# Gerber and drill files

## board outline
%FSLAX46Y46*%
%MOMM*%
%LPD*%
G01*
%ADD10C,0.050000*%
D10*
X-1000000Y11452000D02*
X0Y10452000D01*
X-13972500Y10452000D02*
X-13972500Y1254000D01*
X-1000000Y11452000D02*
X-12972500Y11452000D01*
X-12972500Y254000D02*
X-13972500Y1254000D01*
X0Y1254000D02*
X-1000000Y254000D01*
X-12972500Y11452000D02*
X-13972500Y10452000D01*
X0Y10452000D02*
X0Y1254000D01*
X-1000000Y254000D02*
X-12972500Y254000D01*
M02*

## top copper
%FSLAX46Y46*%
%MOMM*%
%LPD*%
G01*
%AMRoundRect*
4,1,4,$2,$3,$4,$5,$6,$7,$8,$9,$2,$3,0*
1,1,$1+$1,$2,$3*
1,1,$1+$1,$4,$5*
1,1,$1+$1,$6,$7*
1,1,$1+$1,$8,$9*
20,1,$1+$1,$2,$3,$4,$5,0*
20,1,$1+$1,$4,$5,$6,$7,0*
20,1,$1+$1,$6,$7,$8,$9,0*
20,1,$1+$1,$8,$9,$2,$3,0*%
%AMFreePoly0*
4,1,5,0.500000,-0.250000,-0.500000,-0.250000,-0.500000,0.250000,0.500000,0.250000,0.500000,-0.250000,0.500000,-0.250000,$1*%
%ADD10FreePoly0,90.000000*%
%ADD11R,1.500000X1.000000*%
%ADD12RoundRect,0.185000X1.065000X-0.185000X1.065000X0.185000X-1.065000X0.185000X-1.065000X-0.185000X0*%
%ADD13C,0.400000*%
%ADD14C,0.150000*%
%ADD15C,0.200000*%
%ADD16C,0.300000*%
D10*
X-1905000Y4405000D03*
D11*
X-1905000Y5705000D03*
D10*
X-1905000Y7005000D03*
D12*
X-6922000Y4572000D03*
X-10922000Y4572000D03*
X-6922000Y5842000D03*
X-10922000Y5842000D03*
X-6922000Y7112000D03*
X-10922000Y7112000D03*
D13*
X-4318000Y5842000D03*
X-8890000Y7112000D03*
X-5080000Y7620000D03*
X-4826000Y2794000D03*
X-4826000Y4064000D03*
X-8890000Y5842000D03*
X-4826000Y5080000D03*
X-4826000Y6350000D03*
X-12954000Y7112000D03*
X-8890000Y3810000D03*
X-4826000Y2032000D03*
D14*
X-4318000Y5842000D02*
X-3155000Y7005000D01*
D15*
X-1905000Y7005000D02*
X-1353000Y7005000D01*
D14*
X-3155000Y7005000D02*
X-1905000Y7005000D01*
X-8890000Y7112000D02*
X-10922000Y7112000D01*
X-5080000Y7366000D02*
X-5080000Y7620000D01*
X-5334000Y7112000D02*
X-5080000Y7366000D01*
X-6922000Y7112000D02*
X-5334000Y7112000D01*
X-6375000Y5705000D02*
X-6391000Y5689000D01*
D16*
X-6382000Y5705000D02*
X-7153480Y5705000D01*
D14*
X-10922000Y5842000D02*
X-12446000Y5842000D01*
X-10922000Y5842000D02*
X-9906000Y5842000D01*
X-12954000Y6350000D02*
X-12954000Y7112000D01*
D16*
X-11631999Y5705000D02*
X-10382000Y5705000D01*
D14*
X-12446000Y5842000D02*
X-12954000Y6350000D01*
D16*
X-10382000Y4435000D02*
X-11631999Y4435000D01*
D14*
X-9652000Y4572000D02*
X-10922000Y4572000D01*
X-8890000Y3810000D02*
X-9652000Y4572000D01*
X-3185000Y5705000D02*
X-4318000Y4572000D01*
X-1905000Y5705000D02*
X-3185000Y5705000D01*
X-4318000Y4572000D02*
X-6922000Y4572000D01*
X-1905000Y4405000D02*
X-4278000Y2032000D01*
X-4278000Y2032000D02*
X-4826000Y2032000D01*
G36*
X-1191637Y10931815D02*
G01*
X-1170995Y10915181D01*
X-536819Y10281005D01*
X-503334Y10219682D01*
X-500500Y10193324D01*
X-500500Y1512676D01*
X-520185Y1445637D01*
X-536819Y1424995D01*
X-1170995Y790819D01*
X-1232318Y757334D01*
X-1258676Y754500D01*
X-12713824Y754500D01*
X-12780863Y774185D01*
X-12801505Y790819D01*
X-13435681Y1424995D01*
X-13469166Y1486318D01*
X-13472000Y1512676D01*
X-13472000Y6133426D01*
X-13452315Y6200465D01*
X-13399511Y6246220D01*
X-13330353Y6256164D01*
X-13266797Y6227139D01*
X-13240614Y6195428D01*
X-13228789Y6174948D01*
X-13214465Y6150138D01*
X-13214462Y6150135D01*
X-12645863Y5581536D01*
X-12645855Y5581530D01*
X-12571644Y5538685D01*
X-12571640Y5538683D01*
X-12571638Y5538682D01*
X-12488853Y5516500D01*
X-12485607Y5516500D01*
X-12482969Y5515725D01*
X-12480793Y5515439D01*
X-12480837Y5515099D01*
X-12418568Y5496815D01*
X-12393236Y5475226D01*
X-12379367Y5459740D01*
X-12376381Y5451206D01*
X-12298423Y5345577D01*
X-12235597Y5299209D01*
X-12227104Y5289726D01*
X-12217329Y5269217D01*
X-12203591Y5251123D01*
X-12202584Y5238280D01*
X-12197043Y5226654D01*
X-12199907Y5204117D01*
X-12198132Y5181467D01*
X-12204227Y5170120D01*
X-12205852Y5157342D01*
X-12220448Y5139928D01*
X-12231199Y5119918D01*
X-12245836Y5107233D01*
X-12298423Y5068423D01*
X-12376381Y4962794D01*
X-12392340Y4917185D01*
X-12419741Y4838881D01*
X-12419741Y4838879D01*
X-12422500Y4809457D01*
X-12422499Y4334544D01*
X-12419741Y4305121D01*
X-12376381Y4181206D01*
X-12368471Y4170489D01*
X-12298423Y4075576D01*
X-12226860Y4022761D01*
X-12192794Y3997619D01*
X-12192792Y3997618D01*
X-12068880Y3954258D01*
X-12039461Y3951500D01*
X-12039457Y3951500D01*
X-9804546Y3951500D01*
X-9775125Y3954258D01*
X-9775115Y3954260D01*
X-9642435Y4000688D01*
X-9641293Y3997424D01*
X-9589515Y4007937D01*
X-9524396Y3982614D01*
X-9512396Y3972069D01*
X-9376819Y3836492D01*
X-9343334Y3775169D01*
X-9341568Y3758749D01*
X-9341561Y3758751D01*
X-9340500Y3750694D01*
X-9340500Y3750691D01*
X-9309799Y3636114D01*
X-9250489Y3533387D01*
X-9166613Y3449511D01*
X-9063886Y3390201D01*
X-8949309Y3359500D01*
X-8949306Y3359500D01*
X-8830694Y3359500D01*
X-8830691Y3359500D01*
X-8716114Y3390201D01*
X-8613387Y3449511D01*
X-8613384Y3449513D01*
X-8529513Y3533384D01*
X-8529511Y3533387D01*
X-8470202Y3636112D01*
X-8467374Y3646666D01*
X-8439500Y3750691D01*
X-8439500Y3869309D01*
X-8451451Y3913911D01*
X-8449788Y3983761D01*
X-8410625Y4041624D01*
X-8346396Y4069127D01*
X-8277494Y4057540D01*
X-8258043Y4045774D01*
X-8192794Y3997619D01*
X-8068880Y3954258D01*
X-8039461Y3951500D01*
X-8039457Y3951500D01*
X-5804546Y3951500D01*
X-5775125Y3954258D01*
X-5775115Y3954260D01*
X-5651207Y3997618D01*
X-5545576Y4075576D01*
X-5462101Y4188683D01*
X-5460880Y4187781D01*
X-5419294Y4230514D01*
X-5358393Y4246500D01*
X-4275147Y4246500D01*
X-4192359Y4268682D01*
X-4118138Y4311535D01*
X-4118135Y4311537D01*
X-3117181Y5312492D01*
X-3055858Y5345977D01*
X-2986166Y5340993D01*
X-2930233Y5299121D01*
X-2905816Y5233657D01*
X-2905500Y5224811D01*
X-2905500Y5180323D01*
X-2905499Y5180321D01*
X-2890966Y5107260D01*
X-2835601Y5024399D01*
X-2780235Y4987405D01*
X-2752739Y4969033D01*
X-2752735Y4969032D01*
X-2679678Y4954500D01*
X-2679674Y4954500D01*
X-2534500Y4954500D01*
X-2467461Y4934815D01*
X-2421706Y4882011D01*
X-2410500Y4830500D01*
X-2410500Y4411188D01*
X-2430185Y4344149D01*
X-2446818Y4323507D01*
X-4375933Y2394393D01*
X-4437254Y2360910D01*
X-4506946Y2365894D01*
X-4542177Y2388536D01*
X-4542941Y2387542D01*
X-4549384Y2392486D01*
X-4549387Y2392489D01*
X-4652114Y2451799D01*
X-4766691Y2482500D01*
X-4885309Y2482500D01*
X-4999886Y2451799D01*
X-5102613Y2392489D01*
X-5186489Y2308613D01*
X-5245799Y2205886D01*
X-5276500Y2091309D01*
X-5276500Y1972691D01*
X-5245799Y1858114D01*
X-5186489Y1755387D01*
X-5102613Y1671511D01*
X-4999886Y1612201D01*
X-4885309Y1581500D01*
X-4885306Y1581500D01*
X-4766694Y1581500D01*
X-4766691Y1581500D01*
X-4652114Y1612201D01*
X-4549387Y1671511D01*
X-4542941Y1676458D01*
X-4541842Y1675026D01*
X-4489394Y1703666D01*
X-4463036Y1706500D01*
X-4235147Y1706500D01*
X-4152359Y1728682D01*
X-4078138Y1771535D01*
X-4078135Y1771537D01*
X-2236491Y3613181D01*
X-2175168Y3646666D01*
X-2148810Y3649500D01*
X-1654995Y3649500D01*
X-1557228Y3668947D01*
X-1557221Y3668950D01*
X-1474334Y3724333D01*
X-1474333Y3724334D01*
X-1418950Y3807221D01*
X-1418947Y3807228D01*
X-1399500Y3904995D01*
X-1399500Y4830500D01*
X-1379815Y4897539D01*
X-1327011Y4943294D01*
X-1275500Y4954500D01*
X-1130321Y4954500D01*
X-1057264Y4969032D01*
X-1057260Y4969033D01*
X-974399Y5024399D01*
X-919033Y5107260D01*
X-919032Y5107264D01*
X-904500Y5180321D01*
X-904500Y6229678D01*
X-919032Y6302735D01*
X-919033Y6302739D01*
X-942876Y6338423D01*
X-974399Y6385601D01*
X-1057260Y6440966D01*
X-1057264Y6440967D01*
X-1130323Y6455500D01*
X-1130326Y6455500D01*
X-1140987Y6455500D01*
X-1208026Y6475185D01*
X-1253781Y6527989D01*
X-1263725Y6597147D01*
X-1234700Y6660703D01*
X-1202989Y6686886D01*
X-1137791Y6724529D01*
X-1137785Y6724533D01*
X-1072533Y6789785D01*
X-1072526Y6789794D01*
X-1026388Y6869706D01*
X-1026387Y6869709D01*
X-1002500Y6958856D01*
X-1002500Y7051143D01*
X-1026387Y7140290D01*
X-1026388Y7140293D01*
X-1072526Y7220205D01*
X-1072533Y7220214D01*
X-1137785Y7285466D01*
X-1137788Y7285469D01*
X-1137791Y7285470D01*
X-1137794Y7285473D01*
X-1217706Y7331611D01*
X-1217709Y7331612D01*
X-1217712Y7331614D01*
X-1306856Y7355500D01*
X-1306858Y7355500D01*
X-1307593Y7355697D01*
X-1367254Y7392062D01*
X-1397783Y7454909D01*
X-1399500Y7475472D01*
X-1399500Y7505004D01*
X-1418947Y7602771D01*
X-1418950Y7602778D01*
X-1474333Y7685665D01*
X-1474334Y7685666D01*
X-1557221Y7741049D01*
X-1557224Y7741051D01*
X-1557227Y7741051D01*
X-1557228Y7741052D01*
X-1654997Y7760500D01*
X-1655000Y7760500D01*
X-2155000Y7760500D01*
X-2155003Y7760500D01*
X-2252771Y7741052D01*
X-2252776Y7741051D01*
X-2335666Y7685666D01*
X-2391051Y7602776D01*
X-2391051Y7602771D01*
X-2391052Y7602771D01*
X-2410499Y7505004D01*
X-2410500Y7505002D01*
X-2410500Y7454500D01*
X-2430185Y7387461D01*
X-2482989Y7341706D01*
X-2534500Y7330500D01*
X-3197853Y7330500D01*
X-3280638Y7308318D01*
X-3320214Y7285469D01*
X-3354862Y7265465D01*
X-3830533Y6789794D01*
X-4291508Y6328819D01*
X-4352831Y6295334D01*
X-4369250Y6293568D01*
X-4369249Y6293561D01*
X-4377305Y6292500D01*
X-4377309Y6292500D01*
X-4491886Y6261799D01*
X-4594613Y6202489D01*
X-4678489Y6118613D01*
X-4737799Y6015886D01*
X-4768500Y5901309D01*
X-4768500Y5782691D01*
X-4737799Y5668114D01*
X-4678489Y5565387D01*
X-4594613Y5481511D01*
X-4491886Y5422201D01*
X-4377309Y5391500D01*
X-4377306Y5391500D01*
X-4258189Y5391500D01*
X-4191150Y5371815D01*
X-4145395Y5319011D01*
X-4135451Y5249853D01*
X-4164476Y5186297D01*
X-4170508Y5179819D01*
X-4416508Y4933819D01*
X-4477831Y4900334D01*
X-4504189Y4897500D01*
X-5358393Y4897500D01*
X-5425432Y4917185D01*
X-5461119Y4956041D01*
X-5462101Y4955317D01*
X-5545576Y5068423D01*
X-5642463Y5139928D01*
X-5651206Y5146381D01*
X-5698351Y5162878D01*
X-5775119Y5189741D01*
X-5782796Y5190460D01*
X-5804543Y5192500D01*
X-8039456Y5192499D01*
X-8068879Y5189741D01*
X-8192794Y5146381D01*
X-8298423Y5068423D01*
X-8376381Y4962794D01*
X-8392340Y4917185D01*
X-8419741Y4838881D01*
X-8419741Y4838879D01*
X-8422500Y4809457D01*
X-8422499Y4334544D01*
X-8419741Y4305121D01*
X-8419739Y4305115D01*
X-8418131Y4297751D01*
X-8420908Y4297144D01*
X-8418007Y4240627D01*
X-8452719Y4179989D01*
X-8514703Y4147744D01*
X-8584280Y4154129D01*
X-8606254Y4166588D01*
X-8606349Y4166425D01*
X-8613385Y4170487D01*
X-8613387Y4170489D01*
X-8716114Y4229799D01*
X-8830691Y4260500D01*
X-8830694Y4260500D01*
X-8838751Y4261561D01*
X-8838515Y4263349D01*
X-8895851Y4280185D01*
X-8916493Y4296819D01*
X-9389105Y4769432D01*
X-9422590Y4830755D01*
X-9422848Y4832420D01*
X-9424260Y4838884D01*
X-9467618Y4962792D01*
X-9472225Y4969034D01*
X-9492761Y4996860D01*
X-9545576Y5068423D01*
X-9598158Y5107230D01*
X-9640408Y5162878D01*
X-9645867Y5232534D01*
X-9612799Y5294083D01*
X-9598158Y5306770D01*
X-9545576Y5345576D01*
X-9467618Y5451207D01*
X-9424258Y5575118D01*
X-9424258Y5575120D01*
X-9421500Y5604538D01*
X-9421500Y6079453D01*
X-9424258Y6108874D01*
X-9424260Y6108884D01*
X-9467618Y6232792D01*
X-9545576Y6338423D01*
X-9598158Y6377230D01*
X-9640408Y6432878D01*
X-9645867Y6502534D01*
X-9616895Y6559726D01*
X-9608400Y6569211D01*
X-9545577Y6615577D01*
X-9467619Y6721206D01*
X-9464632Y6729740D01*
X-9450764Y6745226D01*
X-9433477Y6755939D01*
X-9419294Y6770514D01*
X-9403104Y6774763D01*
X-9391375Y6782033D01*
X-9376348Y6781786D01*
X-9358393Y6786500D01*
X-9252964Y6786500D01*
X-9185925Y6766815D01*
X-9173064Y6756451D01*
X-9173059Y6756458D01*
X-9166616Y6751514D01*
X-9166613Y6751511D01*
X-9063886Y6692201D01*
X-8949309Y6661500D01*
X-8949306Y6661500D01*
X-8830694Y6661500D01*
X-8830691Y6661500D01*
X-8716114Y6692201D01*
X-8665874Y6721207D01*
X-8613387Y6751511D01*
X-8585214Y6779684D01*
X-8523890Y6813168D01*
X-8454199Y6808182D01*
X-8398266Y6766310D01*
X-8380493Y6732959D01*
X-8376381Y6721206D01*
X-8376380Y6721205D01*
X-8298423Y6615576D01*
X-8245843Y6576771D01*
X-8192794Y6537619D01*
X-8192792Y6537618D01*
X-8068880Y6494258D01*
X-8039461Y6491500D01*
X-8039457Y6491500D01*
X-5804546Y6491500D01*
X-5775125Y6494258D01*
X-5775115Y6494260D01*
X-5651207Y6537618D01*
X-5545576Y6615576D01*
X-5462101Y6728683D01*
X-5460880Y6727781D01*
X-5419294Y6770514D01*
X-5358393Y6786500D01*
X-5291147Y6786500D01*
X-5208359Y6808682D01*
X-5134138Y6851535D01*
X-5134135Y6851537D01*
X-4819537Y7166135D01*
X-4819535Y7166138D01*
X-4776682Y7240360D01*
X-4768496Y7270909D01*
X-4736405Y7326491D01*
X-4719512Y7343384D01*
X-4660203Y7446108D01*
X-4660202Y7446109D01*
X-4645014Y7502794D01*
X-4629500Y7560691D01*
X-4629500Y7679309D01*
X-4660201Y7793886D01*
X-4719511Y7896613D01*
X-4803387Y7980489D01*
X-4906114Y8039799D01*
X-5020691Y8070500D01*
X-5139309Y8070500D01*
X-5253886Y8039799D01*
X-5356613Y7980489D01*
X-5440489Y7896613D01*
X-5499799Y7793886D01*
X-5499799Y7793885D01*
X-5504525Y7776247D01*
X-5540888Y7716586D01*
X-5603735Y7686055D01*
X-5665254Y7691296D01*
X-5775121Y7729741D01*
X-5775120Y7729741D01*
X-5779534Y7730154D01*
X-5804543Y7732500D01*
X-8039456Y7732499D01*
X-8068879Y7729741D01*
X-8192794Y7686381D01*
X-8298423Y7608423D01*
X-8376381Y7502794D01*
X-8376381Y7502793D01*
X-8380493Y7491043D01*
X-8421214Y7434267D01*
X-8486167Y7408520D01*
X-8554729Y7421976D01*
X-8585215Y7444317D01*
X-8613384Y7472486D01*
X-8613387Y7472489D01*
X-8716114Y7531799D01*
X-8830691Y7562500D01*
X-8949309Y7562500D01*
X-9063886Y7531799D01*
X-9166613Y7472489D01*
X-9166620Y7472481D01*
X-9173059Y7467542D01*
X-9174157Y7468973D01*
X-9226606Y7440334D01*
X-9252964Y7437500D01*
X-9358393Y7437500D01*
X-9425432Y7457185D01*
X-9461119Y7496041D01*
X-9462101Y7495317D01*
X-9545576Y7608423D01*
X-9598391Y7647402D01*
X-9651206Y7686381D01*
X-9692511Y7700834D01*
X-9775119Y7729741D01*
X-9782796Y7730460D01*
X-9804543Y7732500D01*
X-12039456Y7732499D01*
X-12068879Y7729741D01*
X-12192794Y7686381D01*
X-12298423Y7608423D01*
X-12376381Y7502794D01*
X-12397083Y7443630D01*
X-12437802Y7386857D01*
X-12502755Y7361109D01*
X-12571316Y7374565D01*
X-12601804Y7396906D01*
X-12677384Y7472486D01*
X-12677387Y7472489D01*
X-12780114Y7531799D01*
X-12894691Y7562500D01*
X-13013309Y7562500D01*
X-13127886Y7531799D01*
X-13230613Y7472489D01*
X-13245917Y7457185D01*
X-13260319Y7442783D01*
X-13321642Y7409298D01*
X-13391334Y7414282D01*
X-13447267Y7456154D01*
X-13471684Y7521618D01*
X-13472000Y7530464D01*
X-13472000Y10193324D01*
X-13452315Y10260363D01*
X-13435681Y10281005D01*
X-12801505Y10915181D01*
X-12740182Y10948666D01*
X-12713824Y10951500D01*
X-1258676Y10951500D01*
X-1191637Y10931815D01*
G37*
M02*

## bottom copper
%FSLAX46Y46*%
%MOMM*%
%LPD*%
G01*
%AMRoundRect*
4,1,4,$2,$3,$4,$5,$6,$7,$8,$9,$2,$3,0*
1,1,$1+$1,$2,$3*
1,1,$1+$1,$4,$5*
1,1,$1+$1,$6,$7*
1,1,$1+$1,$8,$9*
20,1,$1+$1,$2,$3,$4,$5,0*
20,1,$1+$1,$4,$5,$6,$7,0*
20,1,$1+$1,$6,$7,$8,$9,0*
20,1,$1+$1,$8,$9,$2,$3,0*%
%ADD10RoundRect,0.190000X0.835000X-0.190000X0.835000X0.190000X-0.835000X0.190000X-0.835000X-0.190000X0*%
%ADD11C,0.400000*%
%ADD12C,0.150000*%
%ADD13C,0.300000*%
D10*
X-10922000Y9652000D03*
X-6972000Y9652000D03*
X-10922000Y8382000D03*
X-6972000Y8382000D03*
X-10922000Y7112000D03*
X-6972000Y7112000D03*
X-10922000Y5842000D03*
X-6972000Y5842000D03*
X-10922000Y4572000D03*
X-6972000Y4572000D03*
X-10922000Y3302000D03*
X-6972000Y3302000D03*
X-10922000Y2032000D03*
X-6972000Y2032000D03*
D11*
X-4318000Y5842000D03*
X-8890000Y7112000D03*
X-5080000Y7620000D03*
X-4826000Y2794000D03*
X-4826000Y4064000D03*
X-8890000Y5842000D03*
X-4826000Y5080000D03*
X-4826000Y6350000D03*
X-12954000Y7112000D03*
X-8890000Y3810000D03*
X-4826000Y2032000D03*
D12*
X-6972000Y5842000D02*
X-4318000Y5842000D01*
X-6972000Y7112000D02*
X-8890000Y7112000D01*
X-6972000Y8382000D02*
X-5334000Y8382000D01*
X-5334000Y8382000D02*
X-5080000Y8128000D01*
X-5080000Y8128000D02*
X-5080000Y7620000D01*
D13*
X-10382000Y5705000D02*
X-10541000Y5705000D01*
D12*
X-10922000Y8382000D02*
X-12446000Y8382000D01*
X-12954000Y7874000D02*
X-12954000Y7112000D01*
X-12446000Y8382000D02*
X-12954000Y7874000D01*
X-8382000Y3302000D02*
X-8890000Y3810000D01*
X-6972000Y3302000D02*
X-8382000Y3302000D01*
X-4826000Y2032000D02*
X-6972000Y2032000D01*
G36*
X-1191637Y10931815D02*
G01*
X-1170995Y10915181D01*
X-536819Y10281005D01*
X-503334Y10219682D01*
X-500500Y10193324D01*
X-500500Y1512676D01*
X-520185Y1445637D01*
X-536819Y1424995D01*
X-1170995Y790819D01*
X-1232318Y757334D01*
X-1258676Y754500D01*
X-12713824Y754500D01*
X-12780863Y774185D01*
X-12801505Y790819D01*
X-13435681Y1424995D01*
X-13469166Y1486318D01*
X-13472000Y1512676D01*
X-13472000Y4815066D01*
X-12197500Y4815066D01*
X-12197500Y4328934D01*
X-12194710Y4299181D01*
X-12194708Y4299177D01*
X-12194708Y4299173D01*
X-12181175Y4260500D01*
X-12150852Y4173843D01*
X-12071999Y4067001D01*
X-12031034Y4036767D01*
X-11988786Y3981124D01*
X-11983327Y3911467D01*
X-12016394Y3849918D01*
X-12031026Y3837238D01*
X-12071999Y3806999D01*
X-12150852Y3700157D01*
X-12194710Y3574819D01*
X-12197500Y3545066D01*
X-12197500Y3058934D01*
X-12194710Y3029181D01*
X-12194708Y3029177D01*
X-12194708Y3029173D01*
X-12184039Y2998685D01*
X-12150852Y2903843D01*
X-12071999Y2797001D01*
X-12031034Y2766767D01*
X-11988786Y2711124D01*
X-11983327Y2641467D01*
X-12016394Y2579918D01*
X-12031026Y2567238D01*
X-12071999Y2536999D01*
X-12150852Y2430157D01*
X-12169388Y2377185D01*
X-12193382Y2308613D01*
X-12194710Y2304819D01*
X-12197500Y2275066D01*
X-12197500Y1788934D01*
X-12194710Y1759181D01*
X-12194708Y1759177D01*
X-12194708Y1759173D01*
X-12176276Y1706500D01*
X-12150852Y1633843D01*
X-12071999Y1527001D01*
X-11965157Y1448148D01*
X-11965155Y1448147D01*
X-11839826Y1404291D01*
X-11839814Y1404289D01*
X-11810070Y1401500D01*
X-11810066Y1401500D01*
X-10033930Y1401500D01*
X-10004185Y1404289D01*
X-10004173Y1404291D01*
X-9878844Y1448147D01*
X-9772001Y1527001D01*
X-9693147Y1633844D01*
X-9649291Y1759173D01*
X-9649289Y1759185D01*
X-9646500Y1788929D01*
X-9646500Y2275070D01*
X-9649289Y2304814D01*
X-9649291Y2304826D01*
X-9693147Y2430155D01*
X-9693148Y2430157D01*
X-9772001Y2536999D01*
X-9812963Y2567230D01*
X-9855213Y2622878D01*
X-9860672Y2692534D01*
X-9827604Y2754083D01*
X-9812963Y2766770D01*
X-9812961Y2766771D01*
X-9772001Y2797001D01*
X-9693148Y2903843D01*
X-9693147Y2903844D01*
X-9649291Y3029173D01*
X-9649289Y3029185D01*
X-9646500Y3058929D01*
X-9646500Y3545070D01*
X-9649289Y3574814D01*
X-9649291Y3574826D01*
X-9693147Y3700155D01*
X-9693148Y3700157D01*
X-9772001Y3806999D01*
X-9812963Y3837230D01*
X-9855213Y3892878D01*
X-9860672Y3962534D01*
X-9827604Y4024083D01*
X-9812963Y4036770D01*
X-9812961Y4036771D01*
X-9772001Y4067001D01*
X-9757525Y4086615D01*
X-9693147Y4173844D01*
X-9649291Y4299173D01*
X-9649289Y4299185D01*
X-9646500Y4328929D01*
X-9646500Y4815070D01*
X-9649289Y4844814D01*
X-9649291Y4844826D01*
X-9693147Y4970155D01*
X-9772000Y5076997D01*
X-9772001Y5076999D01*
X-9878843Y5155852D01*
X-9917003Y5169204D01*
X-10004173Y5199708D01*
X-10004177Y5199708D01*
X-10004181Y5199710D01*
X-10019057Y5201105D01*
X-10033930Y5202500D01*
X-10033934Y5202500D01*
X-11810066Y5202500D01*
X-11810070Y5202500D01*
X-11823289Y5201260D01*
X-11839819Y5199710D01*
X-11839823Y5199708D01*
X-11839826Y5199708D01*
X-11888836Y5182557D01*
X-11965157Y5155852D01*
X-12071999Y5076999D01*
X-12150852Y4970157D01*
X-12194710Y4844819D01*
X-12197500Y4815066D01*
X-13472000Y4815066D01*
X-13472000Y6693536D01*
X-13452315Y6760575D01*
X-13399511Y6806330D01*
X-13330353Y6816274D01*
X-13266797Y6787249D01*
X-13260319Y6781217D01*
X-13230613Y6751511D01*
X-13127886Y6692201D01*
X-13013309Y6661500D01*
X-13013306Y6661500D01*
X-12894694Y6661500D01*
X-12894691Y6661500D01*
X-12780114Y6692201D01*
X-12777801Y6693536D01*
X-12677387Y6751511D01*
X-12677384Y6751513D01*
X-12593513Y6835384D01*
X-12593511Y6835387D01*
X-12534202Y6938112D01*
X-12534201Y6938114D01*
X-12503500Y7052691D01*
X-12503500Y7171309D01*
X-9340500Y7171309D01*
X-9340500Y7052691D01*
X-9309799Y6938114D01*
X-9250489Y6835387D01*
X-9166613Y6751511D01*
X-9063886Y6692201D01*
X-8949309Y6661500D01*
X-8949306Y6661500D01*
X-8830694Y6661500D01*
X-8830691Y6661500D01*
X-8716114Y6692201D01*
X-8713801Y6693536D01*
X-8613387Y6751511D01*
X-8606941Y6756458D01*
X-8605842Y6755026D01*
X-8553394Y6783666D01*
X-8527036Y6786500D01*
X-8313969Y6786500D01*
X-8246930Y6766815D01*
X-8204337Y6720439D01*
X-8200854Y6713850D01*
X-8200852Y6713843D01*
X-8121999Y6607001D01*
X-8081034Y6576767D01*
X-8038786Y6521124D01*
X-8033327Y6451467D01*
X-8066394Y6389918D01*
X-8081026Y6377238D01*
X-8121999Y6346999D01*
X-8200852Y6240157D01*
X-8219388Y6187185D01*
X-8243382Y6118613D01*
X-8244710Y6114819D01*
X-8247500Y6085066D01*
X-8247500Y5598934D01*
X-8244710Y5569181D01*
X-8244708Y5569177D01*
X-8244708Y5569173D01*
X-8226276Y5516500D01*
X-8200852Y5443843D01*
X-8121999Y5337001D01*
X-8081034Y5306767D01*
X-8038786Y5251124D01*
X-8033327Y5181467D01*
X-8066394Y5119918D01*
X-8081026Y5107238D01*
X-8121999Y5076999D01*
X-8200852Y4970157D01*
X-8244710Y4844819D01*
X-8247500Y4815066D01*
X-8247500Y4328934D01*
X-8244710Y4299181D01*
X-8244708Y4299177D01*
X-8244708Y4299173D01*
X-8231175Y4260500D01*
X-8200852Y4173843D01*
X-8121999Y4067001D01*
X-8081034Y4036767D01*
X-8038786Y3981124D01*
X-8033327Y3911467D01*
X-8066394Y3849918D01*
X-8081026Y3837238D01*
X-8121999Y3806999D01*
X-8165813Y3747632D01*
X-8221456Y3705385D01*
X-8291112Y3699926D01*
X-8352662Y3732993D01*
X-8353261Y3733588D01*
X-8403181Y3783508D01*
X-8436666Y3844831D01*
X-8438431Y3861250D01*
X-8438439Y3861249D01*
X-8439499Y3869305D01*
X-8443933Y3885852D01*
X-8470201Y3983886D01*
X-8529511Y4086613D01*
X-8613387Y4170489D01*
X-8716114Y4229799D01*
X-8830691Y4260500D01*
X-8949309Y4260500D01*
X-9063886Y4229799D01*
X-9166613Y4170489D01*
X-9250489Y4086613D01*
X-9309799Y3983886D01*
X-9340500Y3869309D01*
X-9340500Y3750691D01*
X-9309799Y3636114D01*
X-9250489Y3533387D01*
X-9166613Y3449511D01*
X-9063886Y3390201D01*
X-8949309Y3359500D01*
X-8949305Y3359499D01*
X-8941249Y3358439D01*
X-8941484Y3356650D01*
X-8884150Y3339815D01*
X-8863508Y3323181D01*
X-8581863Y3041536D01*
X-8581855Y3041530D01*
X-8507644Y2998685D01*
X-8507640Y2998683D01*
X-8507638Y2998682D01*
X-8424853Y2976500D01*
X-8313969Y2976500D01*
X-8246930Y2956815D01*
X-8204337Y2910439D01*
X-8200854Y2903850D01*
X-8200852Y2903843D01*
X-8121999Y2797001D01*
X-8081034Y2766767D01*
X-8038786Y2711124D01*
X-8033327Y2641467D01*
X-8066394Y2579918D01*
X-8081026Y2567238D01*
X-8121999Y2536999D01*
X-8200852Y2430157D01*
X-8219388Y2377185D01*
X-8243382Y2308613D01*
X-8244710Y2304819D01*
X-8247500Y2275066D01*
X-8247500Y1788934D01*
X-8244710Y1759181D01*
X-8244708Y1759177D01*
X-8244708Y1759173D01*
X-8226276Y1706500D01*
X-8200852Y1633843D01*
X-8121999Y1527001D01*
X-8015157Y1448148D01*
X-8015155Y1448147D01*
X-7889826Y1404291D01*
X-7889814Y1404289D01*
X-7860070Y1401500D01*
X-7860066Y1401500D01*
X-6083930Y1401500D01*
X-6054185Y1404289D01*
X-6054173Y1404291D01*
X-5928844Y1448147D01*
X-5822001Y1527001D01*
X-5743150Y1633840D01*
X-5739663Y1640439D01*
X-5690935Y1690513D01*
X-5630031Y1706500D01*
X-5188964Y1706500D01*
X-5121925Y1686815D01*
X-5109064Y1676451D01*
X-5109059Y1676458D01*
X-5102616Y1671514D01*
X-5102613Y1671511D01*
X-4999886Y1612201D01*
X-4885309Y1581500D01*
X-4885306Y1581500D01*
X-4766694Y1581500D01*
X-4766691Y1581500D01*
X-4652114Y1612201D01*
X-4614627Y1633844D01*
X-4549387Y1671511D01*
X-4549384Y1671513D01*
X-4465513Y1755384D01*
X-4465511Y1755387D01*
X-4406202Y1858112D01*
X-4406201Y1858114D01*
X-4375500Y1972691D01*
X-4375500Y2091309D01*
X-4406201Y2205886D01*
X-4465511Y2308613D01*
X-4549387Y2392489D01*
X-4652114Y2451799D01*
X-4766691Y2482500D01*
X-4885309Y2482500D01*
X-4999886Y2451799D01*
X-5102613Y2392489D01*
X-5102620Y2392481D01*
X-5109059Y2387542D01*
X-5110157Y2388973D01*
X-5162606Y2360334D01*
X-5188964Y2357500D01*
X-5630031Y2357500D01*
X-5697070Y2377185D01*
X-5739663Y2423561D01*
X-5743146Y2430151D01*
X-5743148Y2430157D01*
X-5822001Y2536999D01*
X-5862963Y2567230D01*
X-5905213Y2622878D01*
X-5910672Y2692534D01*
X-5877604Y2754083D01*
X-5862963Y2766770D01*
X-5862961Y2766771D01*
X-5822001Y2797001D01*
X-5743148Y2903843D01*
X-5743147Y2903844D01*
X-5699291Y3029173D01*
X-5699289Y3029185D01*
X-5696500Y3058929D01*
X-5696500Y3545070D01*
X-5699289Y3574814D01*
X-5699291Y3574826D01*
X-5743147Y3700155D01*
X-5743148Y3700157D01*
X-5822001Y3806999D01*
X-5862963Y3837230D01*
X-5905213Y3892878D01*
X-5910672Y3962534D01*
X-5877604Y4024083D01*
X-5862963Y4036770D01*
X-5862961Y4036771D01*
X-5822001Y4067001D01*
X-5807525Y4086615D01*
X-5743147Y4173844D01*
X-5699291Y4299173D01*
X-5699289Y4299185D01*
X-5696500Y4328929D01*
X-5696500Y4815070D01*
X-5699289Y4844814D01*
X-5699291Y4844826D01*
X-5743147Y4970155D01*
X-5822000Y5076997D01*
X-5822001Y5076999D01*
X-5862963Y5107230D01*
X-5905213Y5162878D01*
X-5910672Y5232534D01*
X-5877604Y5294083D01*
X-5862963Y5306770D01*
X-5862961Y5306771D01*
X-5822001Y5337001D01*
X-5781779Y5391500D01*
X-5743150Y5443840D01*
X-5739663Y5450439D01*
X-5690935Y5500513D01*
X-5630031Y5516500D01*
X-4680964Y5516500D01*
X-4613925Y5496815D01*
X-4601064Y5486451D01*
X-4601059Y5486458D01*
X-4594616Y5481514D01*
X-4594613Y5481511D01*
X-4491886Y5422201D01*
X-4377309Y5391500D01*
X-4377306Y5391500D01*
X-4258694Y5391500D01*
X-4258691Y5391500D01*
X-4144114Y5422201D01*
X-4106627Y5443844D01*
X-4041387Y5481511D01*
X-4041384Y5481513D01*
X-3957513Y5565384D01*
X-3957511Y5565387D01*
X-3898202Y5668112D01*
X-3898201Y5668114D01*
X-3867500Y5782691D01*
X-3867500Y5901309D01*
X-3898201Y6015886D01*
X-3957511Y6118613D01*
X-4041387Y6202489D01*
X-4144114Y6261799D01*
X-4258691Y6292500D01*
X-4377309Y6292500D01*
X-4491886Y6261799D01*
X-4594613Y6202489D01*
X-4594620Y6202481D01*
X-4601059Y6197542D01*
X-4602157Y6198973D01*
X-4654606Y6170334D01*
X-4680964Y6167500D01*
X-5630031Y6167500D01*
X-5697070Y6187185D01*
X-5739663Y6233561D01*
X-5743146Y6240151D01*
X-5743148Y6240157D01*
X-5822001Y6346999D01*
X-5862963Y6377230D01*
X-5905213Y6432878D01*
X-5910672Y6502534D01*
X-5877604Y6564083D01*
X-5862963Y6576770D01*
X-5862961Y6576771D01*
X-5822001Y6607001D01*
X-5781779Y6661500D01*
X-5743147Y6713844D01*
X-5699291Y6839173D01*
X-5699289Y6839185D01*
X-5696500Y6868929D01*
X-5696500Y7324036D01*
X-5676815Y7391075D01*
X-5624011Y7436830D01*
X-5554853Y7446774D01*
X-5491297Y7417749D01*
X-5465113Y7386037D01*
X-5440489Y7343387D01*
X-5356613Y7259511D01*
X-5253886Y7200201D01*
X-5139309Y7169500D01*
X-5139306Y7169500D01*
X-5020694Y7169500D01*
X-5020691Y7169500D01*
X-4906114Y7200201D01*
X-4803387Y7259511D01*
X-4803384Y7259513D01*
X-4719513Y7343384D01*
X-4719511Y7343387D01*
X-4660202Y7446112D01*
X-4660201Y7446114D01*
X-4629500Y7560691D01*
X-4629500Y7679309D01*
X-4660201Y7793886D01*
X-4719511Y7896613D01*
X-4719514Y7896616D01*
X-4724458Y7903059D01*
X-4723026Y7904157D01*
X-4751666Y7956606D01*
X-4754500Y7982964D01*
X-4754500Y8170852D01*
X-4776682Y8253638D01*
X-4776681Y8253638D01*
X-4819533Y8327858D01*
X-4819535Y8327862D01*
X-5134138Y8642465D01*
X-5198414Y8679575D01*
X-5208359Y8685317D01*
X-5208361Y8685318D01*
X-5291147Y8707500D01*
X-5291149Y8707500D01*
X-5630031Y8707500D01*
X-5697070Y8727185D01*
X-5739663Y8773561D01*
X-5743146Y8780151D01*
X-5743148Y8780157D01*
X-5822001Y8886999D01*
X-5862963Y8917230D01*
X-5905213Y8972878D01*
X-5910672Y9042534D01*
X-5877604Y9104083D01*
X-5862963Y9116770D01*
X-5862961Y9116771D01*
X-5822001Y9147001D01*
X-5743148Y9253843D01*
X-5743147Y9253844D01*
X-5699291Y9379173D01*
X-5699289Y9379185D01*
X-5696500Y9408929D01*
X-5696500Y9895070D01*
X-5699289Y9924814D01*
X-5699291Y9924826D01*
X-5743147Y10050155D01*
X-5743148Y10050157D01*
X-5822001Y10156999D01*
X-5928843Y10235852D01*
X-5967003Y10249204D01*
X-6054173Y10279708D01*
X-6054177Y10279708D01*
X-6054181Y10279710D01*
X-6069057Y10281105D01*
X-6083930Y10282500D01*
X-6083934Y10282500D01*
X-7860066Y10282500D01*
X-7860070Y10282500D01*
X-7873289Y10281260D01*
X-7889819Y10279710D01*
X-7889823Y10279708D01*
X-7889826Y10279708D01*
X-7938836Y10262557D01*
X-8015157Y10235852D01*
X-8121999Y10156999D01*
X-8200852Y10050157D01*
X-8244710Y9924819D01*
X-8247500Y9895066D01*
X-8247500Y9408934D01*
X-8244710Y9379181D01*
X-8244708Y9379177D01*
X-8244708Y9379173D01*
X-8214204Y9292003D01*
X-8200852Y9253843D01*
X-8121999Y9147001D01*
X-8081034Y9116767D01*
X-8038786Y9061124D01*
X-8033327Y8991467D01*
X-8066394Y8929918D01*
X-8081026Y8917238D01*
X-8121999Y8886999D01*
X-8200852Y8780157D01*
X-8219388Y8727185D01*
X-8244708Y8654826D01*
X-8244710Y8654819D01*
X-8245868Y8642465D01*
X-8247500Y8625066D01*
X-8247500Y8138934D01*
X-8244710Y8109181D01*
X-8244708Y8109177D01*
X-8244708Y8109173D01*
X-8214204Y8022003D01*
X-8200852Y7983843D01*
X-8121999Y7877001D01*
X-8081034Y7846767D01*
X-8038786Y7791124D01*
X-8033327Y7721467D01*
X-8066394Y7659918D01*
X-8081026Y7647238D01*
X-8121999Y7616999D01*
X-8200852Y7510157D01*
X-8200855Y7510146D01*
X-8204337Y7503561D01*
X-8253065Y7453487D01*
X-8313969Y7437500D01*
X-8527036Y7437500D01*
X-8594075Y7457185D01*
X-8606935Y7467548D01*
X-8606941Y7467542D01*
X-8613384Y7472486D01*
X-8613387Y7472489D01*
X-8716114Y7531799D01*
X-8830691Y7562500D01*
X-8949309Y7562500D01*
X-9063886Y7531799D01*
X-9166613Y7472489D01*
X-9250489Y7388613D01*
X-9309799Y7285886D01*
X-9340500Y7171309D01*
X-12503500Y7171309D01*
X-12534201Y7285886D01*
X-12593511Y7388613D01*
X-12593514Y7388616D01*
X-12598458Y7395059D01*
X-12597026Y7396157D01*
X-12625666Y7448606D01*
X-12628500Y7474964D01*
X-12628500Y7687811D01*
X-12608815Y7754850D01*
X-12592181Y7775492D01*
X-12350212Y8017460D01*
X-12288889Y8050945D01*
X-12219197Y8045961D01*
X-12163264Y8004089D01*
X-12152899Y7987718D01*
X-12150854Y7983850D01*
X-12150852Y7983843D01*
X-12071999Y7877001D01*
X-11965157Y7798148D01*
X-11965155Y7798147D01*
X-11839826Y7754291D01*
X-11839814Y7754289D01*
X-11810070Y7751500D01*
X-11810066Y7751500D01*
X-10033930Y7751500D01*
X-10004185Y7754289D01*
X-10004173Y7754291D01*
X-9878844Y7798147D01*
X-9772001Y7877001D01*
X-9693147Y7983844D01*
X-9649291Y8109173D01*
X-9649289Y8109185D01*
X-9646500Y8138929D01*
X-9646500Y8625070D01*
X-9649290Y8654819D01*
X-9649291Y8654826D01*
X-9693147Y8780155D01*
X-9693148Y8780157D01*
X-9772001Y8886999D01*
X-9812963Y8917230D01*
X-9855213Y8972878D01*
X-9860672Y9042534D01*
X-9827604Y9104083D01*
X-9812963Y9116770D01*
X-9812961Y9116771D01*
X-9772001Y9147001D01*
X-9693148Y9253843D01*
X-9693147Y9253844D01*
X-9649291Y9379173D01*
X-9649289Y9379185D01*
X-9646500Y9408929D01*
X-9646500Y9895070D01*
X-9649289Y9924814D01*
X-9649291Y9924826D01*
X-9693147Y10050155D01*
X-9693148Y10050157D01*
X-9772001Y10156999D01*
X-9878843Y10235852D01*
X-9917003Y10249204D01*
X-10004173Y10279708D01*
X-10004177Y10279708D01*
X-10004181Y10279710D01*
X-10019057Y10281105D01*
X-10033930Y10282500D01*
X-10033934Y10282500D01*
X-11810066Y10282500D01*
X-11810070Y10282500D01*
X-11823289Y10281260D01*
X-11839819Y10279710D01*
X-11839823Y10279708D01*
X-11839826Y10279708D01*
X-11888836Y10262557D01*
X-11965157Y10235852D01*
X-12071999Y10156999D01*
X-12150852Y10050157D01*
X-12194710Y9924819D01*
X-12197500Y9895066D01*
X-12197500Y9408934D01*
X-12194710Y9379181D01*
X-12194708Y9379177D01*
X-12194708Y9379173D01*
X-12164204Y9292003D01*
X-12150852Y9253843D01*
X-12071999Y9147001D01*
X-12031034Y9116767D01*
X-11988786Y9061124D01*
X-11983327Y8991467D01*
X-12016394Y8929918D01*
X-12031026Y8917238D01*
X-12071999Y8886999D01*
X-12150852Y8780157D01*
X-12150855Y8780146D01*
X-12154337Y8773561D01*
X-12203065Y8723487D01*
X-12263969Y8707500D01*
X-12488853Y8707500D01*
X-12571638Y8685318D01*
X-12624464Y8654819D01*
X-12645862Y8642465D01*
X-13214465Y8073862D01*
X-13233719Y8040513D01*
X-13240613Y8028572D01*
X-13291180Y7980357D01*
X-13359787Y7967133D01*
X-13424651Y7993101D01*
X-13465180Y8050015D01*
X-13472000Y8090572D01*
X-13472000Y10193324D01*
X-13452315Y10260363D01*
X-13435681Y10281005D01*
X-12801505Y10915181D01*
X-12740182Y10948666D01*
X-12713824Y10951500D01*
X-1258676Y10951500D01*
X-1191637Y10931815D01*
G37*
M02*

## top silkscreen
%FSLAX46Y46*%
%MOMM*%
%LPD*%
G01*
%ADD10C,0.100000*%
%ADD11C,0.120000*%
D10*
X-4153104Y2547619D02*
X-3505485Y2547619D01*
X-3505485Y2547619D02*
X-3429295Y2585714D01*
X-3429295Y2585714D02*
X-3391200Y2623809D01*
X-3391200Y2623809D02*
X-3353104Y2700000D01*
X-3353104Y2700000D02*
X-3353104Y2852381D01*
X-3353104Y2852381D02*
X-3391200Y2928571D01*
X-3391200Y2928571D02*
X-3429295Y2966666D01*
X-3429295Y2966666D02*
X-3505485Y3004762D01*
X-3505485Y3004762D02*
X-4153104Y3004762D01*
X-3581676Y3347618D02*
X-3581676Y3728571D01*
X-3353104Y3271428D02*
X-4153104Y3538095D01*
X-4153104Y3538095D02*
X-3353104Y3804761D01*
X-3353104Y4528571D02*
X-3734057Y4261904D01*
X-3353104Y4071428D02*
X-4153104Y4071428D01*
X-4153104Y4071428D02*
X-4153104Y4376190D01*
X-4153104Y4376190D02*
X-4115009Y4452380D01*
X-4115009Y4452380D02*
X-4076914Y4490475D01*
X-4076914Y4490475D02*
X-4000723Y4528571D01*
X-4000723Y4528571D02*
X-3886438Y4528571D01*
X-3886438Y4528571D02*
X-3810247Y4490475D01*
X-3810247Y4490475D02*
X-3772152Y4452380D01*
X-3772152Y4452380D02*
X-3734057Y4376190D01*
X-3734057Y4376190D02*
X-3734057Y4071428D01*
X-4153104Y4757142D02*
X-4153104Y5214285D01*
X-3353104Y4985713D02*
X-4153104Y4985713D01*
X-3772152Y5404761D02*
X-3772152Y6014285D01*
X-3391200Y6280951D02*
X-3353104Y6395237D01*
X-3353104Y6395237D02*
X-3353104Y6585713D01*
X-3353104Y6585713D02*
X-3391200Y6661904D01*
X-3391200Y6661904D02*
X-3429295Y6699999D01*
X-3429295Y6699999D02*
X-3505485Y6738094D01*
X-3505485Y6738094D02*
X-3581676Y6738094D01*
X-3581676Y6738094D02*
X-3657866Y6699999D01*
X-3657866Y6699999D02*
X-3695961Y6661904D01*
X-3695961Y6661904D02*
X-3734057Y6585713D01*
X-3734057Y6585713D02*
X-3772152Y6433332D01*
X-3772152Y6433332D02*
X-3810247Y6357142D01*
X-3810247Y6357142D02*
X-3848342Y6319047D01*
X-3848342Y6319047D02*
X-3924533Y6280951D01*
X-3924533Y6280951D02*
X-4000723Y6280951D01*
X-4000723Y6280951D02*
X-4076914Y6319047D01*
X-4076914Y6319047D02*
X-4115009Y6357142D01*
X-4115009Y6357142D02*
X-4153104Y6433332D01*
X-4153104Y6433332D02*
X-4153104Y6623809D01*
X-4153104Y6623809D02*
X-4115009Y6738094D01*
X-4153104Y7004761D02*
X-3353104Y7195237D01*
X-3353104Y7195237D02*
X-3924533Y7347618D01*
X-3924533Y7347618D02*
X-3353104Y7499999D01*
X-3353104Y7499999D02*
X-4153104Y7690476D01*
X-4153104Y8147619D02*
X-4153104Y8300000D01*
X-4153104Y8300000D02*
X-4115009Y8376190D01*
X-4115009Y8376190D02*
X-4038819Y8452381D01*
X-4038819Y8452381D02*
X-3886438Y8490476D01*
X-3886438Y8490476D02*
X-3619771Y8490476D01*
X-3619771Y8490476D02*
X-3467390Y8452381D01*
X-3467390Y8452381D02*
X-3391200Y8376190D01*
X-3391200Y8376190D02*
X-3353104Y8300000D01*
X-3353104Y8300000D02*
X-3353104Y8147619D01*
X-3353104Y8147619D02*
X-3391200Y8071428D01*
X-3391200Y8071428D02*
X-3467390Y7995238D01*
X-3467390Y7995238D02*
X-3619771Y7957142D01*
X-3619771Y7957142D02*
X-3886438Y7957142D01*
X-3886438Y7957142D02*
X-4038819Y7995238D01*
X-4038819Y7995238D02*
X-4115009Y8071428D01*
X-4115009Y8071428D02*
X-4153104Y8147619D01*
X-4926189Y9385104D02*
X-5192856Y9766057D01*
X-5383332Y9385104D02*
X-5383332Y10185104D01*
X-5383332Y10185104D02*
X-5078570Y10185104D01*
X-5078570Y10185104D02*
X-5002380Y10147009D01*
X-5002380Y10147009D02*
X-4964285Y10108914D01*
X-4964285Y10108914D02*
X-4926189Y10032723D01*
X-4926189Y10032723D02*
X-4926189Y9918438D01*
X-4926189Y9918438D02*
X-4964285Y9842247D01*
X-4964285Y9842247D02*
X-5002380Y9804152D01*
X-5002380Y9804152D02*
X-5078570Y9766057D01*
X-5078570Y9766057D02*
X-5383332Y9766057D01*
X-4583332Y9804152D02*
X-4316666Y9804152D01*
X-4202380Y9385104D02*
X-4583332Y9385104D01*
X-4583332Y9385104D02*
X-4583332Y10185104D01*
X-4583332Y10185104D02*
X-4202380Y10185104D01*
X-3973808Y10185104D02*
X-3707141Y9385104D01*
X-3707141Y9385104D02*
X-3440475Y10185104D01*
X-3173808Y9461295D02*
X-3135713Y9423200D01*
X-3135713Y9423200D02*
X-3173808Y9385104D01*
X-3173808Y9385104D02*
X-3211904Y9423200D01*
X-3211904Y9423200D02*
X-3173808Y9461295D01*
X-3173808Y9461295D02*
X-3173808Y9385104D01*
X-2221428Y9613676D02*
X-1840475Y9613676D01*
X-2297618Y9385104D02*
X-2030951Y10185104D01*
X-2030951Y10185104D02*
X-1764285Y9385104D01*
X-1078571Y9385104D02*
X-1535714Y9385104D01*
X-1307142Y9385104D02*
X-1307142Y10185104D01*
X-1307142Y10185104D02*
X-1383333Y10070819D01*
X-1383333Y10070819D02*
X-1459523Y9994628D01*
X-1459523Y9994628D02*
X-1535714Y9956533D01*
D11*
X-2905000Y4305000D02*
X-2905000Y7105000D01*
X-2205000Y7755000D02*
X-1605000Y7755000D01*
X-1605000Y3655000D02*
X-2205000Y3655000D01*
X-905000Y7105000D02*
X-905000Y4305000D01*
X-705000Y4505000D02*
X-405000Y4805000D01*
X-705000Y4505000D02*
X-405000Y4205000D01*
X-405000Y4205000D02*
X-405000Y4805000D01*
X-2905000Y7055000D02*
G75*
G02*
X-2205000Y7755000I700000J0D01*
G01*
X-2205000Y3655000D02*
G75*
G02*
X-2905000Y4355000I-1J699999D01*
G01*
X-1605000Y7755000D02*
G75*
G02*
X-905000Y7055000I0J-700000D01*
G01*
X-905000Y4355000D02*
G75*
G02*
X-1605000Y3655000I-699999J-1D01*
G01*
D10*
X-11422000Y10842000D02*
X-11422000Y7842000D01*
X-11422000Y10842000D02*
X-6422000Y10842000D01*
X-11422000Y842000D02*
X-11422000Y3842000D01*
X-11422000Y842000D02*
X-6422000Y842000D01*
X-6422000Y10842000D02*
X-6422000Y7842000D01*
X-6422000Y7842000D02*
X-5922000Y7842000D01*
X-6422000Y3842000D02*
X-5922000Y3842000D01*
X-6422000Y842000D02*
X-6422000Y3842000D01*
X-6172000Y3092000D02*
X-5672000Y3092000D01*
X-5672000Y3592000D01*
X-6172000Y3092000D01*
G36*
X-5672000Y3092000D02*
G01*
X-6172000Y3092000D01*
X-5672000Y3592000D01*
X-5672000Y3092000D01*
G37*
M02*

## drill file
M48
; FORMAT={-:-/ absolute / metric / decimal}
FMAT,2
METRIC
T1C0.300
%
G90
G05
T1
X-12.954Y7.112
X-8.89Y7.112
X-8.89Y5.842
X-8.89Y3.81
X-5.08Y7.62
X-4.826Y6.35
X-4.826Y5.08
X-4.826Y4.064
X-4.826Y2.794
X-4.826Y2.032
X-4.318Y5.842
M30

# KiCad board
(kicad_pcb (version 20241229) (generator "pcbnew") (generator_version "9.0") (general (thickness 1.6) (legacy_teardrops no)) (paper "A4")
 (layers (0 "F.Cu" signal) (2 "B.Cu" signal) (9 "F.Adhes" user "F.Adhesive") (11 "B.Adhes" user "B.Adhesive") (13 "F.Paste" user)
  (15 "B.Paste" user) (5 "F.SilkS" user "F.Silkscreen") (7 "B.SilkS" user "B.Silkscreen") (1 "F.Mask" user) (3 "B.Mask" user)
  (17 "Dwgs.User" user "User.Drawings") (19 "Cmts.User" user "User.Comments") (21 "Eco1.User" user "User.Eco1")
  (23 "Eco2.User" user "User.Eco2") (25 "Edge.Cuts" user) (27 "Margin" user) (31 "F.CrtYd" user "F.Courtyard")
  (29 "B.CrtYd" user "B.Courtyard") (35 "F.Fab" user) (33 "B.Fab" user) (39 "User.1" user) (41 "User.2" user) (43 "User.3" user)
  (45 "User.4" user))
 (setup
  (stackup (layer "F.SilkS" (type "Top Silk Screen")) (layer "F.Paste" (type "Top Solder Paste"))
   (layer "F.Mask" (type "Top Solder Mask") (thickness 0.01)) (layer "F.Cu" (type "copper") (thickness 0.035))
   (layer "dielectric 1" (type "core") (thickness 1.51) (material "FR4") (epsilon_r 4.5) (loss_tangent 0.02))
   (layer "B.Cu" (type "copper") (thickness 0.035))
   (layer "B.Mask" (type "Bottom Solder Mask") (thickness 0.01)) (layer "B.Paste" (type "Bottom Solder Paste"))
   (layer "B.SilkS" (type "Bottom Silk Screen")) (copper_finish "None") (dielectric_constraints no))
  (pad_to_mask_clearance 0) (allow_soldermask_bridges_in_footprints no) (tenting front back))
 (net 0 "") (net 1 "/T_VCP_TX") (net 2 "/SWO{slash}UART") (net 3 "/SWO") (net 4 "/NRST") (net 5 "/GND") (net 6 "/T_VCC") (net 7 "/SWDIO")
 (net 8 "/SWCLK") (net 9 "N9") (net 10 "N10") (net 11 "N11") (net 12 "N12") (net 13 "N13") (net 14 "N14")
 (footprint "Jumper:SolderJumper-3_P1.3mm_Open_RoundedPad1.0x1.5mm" (layer "F.Cu") (at -1.905 -5.705 90)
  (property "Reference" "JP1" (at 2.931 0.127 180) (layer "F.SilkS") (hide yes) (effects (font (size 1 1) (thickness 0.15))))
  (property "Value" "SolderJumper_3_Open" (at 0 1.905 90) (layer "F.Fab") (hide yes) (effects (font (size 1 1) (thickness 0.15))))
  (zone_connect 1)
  (fp_line (start -1.4 -1) (end 1.4 -1) (stroke (width 0.12) (type solid)) (layer "F.SilkS"))
  (fp_line (start 2.05 -0.3) (end 2.05 0.3) (stroke (width 0.12) (type solid)) (layer "F.SilkS"))
  (fp_line (start -2.05 0.3) (end -2.05 -0.3) (stroke (width 0.12) (type solid)) (layer "F.SilkS"))
  (fp_line (start 1.4 1) (end -1.4 1) (stroke (width 0.12) (type solid)) (layer "F.SilkS"))
  (fp_line (start -1.2 1.2) (end -0.9 1.5) (stroke (width 0.12) (type solid)) (layer "F.SilkS"))
  (fp_line (start -1.2 1.2) (end -1.5 1.5) (stroke (width 0.12) (type solid)) (layer "F.SilkS"))
  (fp_line (start -1.5 1.5) (end -0.9 1.5) (stroke (width 0.12) (type solid)) (layer "F.SilkS"))
  (fp_arc (start 1.35 -1) (mid 1.844975 -0.794975) (end 2.05 -0.3) (stroke (width 0.12) (type solid)) (layer "F.SilkS"))
  (fp_arc (start -2.05 -0.3) (mid -1.844975 -0.794975) (end -1.35 -1) (stroke (width 0.12) (type solid)) (layer "F.SilkS"))
  (fp_arc (start 2.05 0.3) (mid 1.844975 0.794975) (end 1.35 1) (stroke (width 0.12) (type solid)) (layer "F.SilkS"))
  (fp_arc (start -1.35 1) (mid -1.844975 0.794975) (end -2.05 0.3) (stroke (width 0.12) (type solid)) (layer "F.SilkS"))
  (pad "1" smd custom (at -1.3 0 90) (size 1 0.5) (layers "F.Cu" "F.Mask") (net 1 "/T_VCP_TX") (zone_connect 2) (thermal_bridge_angle 45)
   (options (clearance outline) (anchor rect)) (primitives))
  (pad "2" smd rect (at 0 0 90) (size 1 1.5) (layers "F.Cu" "F.Mask") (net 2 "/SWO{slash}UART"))
  (pad "3" smd custom (at 1.3 0 90) (size 1 0.5) (layers "F.Cu" "F.Mask") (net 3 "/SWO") (zone_connect 2) (thermal_bridge_angle 45)
   (options (clearance outline) (anchor rect)) (primitives)))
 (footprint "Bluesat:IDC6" (layer "F.Cu") (at -8.922 -5.842 90)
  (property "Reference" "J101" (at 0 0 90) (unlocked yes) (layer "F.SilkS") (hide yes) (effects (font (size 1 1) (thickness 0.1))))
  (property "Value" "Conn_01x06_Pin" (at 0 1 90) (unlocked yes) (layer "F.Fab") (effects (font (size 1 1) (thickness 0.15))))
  (fp_line (start 5 -2.5) (end 2 -2.5) (stroke (width 0.1) (type default)) (layer "F.SilkS"))
  (fp_line (start 5 -2.5) (end 5 2.5) (stroke (width 0.1) (type default)) (layer "F.SilkS"))
  (fp_line (start -5 -2.5) (end -2 -2.5) (stroke (width 0.1) (type default)) (layer "F.SilkS"))
  (fp_line (start -5 -2.5) (end -5 2.5) (stroke (width 0.1) (type default)) (layer "F.SilkS"))
  (fp_line (start 5 2.5) (end 2 2.5) (stroke (width 0.1) (type default)) (layer "F.SilkS"))
  (fp_line (start 2 2.5) (end 2 3) (stroke (width 0.1) (type default)) (layer "F.SilkS"))
  (fp_line (start -2 2.5) (end -2 3) (stroke (width 0.1) (type default)) (layer "F.SilkS"))
  (fp_line (start -5 2.5) (end -2 2.5) (stroke (width 0.1) (type default)) (layer "F.SilkS"))
  (fp_poly (pts (xy -2.75 2.75) (xy -2.75 3.25) (xy -2.25 3.25)) (stroke (width 0.1) (type solid)) (fill yes) (layer "F.SilkS"))
  (pad "1" smd roundrect (at -1.27 2 90) (size 0.74 2.5) (layers "F.Cu" "F.Mask" "F.Paste") (roundrect_rratio 0.25)
   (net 2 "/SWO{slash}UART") (thermal_bridge_angle 45))
  (pad "2" smd roundrect (at -1.27 -2 90) (size 0.74 2.5) (layers "F.Cu" "F.Mask" "F.Paste") (roundrect_rratio 0.25) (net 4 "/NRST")
   (thermal_bridge_angle 45))
  (pad "3" smd roundrect (at 0 2 90) (size 0.74 2.5) (layers "F.Cu" "F.Mask" "F.Paste") (roundrect_rratio 0.25) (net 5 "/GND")
   (thermal_bridge_angle 45))
  (pad "4" smd roundrect (at 0 -2 90) (size 0.74 2.5) (layers "F.Cu" "F.Mask" "F.Paste") (roundrect_rratio 0.25) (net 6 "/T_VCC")
   (thermal_bridge_angle 45))
  (pad "5" smd roundrect (at 1.27 2 90) (size 0.74 2.5) (layers "F.Cu" "F.Mask" "F.Paste") (roundrect_rratio 0.25) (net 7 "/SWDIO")
   (thermal_bridge_angle 45))
  (pad "6" smd roundrect (at 1.27 -2 90) (size 0.74 2.5) (layers "F.Cu" "F.Mask" "F.Paste") (roundrect_rratio 0.25) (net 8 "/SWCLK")
   (thermal_bridge_angle 45)))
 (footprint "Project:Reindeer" (layer "B.Cu") (at -2.5 -3.75 180)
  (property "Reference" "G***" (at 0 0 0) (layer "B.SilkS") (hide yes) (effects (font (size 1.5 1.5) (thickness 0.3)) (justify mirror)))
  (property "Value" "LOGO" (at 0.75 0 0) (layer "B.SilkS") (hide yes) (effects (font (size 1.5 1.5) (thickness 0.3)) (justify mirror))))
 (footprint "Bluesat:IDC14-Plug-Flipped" (layer "B.Cu") (at -8.947 -5.842 90)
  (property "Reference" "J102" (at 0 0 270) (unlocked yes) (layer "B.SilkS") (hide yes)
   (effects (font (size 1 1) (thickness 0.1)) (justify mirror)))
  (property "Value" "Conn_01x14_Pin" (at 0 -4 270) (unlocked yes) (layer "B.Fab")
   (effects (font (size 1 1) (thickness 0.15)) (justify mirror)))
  (pad "1" smd roundrect (at 3.81 -1.975 90) (size 0.76 2.05) (layers "B.Cu" "B.Mask" "B.Paste") (roundrect_rratio 0.25) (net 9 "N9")
   (thermal_bridge_angle 45))
  (pad "2" smd roundrect (at 3.81 1.975 90) (size 0.76 2.05) (layers "B.Cu" "B.Mask" "B.Paste") (roundrect_rratio 0.25) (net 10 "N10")
   (thermal_bridge_angle 45))
  (pad "3" smd roundrect (at 2.54 -1.975 90) (size 0.76 2.05) (layers "B.Cu" "B.Mask" "B.Paste") (roundrect_rratio 0.25) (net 6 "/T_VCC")
   (thermal_bridge_angle 45))
  (pad "4" smd roundrect (at 2.54 1.975 90) (size 0.76 2.05) (layers "B.Cu" "B.Mask" "B.Paste") (roundrect_rratio 0.25) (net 7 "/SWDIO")
   (thermal_bridge_angle 45))
  (pad "5" smd roundrect (at 1.27 -1.975 90) (size 0.76 2.05) (layers "B.Cu" "B.Mask" "B.Paste") (roundrect_rratio 0.25) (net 5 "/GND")
   (thermal_bridge_angle 45))
  (pad "6" smd roundrect (at 1.27 1.975 90) (size 0.76 2.05) (layers "B.Cu" "B.Mask" "B.Paste") (roundrect_rratio 0.25) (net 8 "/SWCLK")
   (thermal_bridge_angle 45))
  (pad "7" smd roundrect (at 0 -1.975 90) (size 0.76 2.05) (layers "B.Cu" "B.Mask" "B.Paste") (roundrect_rratio 0.25) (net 5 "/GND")
   (thermal_bridge_angle 45))
  (pad "8" smd roundrect (at 0 1.975 90) (size 0.76 2.05) (layers "B.Cu" "B.Mask" "B.Paste") (roundrect_rratio 0.25) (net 3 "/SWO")
   (thermal_bridge_angle 45))
  (pad "9" smd roundrect (at -1.27 -1.975 90) (size 0.76 2.05) (layers "B.Cu" "B.Mask" "B.Paste") (roundrect_rratio 0.25) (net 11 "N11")
   (thermal_bridge_angle 45))
  (pad "10" smd roundrect (at -1.27 1.975 90) (size 0.76 2.05) (layers "B.Cu" "B.Mask" "B.Paste") (roundrect_rratio 0.25) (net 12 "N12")
   (thermal_bridge_angle 45))
  (pad "11" smd roundrect (at -2.54 -1.975 90) (size 0.76 2.05) (layers "B.Cu" "B.Mask" "B.Paste") (roundrect_rratio 0.25) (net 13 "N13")
   (thermal_bridge_angle 45))
  (pad "12" smd roundrect (at -2.54 1.975 90) (size 0.76 2.05) (layers "B.Cu" "B.Mask" "B.Paste") (roundrect_rratio 0.25) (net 4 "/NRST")
   (thermal_bridge_angle 45))
  (pad "13" smd roundrect (at -3.81 -1.975 90) (size 0.76 2.05) (layers "B.Cu" "B.Mask" "B.Paste") (roundrect_rratio 0.25) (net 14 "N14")
   (thermal_bridge_angle 45))
  (pad "14" smd roundrect (at -3.81 1.975 90) (size 0.76 2.05) (layers "B.Cu" "B.Mask" "B.Paste") (roundrect_rratio 0.25)
   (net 1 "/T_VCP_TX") (thermal_bridge_angle 45)))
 (gr_line (start -1 -11.452) (end 0 -10.452) (stroke (width 0.05) (type default)) (layer "Edge.Cuts"))
 (gr_line (start -13.9725 -10.452) (end -13.9725 -1.254) (stroke (width 0.05) (type default)) (layer "Edge.Cuts"))
 (gr_line (start -1 -11.452) (end -12.9725 -11.452) (stroke (width 0.05) (type default)) (layer "Edge.Cuts"))
 (gr_line (start -12.9725 -0.254) (end -13.9725 -1.254) (stroke (width 0.05) (type default)) (layer "Edge.Cuts"))
 (gr_line (start 0 -1.254) (end -1 -0.254) (stroke (width 0.05) (type default)) (layer "Edge.Cuts"))
 (gr_line (start -12.9725 -11.452) (end -13.9725 -10.452) (stroke (width 0.05) (type default)) (layer "Edge.Cuts"))
 (gr_line (start 0 -10.452) (end 0 -1.254) (stroke (width 0.05) (type default)) (layer "Edge.Cuts"))
 (gr_line (start -1 -0.254) (end -12.9725 -0.254) (stroke (width 0.05) (type default)) (layer "Edge.Cuts"))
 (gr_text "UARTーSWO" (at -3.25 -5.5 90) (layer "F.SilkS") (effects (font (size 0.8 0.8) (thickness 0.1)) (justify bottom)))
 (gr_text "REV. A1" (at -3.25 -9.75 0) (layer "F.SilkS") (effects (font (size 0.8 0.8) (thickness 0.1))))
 (segment (start -4.318 -5.842) (end -3.155 -7.005) (width 0.15) (layer "F.Cu") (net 3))
 (segment (start -1.905 -7.005) (end -1.353 -7.005) (width 0.2) (layer "F.Cu") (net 3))
 (segment (start -3.155 -7.005) (end -1.905 -7.005) (width 0.15) (layer "F.Cu") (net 3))
 (via (at -4.318 -5.842) (size 0.4) (drill 0.3) (layers "F.Cu" "B.Cu") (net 3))
 (segment (start -6.972 -5.842) (end -4.318 -5.842) (width 0.15) (layer "B.Cu") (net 3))
 (segment (start -8.89 -7.112) (end -10.922 -7.112) (width 0.15) (layer "F.Cu") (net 8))
 (via (at -8.89 -7.112) (size 0.4) (drill 0.3) (layers "F.Cu" "B.Cu") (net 8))
 (segment (start -6.972 -7.112) (end -8.89 -7.112) (width 0.15) (layer "B.Cu") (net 8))
 (segment (start -5.08 -7.366) (end -5.08 -7.62) (width 0.15) (layer "F.Cu") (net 7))
 (segment (start -5.334 -7.112) (end -5.08 -7.366) (width 0.15) (layer "F.Cu") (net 7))
 (segment (start -6.922 -7.112) (end -5.334 -7.112) (width 0.15) (layer "F.Cu") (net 7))
 (via (at -5.08 -7.62) (size 0.4) (drill 0.3) (layers "F.Cu" "B.Cu") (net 7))
 (segment (start -6.972 -8.382) (end -5.334 -8.382) (width 0.15) (layer "B.Cu") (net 7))
 (segment (start -5.334 -8.382) (end -5.08 -8.128) (width 0.15) (layer "B.Cu") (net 7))
 (segment (start -5.08 -8.128) (end -5.08 -7.62) (width 0.15) (layer "B.Cu") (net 7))
 (segment (start -6.375 -5.705) (end -6.391 -5.689) (width 0.15) (layer "F.Cu") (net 5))
 (segment (start -6.382 -5.705) (end -7.15348 -5.705) (width 0.3) (layer "F.Cu") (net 5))
 (via (at -4.826 -2.794) (size 0.4) (drill 0.3) (layers "F.Cu" "B.Cu") (free yes) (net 5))
 (via (at -4.826 -4.064) (size 0.4) (drill 0.3) (layers "F.Cu" "B.Cu") (free yes) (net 5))
 (via (at -8.89 -5.842) (size 0.4) (drill 0.3) (layers "F.Cu" "B.Cu") (free yes) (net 5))
 (via (at -4.826 -5.08) (size 0.4) (drill 0.3) (layers "F.Cu" "B.Cu") (free yes) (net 5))
 (via (at -4.826 -6.35) (size 0.4) (drill 0.3) (layers "F.Cu" "B.Cu") (free yes) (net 5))
 (segment (start -10.382 -5.705) (end -10.541 -5.705) (width 0.3) (layer "B.Cu") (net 5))
 (segment (start -10.922 -5.842) (end -12.446 -5.842) (width 0.15) (layer "F.Cu") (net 6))
 (segment (start -10.922 -5.842) (end -9.906 -5.842) (width 0.15) (layer "F.Cu") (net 6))
 (segment (start -12.954 -6.35) (end -12.954 -7.112) (width 0.15) (layer "F.Cu") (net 6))
 (segment (start -11.631999 -5.705) (end -10.382 -5.705) (width 0.3) (layer "F.Cu") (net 6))
 (segment (start -12.446 -5.842) (end -12.954 -6.35) (width 0.15) (layer "F.Cu") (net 6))
 (via (at -12.954 -7.112) (size 0.4) (drill 0.3) (layers "F.Cu" "B.Cu") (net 6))
 (segment (start -10.922 -8.382) (end -12.446 -8.382) (width 0.15) (layer "B.Cu") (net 6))
 (segment (start -12.954 -7.874) (end -12.954 -7.112) (width 0.15) (layer "B.Cu") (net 6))
 (segment (start -12.446 -8.382) (end -12.954 -7.874) (width 0.15) (layer "B.Cu") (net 6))
 (segment (start -10.382 -4.435) (end -11.631999 -4.435) (width 0.3) (layer "F.Cu") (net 4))
 (segment (start -9.652 -4.572) (end -10.922 -4.572) (width 0.15) (layer "F.Cu") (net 4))
 (segment (start -8.89 -3.81) (end -9.652 -4.572) (width 0.15) (layer "F.Cu") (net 4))
 (via (at -8.89 -3.81) (size 0.4) (drill 0.3) (layers "F.Cu" "B.Cu") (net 4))
 (segment (start -8.382 -3.302) (end -8.89 -3.81) (width 0.15) (layer "B.Cu") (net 4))
 (segment (start -6.972 -3.302) (end -8.382 -3.302) (width 0.15) (layer "B.Cu") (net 4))
 (segment (start -3.185 -5.705) (end -4.318 -4.572) (width 0.15) (layer "F.Cu") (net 2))
 (segment (start -1.905 -5.705) (end -3.185 -5.705) (width 0.15) (layer "F.Cu") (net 2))
 (segment (start -4.318 -4.572) (end -6.922 -4.572) (width 0.15) (layer "F.Cu") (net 2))
 (segment (start -1.905 -4.405) (end -4.278 -2.032) (width 0.15) (layer "F.Cu") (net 1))
 (segment (start -4.278 -2.032) (end -4.826 -2.032) (width 0.15) (layer "F.Cu") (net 1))
 (via (at -4.826 -2.032) (size 0.4) (drill 0.3) (layers "F.Cu" "B.Cu") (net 1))
 (segment (start -4.826 -2.032) (end -6.972 -2.032) (width 0.15) (layer "B.Cu") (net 1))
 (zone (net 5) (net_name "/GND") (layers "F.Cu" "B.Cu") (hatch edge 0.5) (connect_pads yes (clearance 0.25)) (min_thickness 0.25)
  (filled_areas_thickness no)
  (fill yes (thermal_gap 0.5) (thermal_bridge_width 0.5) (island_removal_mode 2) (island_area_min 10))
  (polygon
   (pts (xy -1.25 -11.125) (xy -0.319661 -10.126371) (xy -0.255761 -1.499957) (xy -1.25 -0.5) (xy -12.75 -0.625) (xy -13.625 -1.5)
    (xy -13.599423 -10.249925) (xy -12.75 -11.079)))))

